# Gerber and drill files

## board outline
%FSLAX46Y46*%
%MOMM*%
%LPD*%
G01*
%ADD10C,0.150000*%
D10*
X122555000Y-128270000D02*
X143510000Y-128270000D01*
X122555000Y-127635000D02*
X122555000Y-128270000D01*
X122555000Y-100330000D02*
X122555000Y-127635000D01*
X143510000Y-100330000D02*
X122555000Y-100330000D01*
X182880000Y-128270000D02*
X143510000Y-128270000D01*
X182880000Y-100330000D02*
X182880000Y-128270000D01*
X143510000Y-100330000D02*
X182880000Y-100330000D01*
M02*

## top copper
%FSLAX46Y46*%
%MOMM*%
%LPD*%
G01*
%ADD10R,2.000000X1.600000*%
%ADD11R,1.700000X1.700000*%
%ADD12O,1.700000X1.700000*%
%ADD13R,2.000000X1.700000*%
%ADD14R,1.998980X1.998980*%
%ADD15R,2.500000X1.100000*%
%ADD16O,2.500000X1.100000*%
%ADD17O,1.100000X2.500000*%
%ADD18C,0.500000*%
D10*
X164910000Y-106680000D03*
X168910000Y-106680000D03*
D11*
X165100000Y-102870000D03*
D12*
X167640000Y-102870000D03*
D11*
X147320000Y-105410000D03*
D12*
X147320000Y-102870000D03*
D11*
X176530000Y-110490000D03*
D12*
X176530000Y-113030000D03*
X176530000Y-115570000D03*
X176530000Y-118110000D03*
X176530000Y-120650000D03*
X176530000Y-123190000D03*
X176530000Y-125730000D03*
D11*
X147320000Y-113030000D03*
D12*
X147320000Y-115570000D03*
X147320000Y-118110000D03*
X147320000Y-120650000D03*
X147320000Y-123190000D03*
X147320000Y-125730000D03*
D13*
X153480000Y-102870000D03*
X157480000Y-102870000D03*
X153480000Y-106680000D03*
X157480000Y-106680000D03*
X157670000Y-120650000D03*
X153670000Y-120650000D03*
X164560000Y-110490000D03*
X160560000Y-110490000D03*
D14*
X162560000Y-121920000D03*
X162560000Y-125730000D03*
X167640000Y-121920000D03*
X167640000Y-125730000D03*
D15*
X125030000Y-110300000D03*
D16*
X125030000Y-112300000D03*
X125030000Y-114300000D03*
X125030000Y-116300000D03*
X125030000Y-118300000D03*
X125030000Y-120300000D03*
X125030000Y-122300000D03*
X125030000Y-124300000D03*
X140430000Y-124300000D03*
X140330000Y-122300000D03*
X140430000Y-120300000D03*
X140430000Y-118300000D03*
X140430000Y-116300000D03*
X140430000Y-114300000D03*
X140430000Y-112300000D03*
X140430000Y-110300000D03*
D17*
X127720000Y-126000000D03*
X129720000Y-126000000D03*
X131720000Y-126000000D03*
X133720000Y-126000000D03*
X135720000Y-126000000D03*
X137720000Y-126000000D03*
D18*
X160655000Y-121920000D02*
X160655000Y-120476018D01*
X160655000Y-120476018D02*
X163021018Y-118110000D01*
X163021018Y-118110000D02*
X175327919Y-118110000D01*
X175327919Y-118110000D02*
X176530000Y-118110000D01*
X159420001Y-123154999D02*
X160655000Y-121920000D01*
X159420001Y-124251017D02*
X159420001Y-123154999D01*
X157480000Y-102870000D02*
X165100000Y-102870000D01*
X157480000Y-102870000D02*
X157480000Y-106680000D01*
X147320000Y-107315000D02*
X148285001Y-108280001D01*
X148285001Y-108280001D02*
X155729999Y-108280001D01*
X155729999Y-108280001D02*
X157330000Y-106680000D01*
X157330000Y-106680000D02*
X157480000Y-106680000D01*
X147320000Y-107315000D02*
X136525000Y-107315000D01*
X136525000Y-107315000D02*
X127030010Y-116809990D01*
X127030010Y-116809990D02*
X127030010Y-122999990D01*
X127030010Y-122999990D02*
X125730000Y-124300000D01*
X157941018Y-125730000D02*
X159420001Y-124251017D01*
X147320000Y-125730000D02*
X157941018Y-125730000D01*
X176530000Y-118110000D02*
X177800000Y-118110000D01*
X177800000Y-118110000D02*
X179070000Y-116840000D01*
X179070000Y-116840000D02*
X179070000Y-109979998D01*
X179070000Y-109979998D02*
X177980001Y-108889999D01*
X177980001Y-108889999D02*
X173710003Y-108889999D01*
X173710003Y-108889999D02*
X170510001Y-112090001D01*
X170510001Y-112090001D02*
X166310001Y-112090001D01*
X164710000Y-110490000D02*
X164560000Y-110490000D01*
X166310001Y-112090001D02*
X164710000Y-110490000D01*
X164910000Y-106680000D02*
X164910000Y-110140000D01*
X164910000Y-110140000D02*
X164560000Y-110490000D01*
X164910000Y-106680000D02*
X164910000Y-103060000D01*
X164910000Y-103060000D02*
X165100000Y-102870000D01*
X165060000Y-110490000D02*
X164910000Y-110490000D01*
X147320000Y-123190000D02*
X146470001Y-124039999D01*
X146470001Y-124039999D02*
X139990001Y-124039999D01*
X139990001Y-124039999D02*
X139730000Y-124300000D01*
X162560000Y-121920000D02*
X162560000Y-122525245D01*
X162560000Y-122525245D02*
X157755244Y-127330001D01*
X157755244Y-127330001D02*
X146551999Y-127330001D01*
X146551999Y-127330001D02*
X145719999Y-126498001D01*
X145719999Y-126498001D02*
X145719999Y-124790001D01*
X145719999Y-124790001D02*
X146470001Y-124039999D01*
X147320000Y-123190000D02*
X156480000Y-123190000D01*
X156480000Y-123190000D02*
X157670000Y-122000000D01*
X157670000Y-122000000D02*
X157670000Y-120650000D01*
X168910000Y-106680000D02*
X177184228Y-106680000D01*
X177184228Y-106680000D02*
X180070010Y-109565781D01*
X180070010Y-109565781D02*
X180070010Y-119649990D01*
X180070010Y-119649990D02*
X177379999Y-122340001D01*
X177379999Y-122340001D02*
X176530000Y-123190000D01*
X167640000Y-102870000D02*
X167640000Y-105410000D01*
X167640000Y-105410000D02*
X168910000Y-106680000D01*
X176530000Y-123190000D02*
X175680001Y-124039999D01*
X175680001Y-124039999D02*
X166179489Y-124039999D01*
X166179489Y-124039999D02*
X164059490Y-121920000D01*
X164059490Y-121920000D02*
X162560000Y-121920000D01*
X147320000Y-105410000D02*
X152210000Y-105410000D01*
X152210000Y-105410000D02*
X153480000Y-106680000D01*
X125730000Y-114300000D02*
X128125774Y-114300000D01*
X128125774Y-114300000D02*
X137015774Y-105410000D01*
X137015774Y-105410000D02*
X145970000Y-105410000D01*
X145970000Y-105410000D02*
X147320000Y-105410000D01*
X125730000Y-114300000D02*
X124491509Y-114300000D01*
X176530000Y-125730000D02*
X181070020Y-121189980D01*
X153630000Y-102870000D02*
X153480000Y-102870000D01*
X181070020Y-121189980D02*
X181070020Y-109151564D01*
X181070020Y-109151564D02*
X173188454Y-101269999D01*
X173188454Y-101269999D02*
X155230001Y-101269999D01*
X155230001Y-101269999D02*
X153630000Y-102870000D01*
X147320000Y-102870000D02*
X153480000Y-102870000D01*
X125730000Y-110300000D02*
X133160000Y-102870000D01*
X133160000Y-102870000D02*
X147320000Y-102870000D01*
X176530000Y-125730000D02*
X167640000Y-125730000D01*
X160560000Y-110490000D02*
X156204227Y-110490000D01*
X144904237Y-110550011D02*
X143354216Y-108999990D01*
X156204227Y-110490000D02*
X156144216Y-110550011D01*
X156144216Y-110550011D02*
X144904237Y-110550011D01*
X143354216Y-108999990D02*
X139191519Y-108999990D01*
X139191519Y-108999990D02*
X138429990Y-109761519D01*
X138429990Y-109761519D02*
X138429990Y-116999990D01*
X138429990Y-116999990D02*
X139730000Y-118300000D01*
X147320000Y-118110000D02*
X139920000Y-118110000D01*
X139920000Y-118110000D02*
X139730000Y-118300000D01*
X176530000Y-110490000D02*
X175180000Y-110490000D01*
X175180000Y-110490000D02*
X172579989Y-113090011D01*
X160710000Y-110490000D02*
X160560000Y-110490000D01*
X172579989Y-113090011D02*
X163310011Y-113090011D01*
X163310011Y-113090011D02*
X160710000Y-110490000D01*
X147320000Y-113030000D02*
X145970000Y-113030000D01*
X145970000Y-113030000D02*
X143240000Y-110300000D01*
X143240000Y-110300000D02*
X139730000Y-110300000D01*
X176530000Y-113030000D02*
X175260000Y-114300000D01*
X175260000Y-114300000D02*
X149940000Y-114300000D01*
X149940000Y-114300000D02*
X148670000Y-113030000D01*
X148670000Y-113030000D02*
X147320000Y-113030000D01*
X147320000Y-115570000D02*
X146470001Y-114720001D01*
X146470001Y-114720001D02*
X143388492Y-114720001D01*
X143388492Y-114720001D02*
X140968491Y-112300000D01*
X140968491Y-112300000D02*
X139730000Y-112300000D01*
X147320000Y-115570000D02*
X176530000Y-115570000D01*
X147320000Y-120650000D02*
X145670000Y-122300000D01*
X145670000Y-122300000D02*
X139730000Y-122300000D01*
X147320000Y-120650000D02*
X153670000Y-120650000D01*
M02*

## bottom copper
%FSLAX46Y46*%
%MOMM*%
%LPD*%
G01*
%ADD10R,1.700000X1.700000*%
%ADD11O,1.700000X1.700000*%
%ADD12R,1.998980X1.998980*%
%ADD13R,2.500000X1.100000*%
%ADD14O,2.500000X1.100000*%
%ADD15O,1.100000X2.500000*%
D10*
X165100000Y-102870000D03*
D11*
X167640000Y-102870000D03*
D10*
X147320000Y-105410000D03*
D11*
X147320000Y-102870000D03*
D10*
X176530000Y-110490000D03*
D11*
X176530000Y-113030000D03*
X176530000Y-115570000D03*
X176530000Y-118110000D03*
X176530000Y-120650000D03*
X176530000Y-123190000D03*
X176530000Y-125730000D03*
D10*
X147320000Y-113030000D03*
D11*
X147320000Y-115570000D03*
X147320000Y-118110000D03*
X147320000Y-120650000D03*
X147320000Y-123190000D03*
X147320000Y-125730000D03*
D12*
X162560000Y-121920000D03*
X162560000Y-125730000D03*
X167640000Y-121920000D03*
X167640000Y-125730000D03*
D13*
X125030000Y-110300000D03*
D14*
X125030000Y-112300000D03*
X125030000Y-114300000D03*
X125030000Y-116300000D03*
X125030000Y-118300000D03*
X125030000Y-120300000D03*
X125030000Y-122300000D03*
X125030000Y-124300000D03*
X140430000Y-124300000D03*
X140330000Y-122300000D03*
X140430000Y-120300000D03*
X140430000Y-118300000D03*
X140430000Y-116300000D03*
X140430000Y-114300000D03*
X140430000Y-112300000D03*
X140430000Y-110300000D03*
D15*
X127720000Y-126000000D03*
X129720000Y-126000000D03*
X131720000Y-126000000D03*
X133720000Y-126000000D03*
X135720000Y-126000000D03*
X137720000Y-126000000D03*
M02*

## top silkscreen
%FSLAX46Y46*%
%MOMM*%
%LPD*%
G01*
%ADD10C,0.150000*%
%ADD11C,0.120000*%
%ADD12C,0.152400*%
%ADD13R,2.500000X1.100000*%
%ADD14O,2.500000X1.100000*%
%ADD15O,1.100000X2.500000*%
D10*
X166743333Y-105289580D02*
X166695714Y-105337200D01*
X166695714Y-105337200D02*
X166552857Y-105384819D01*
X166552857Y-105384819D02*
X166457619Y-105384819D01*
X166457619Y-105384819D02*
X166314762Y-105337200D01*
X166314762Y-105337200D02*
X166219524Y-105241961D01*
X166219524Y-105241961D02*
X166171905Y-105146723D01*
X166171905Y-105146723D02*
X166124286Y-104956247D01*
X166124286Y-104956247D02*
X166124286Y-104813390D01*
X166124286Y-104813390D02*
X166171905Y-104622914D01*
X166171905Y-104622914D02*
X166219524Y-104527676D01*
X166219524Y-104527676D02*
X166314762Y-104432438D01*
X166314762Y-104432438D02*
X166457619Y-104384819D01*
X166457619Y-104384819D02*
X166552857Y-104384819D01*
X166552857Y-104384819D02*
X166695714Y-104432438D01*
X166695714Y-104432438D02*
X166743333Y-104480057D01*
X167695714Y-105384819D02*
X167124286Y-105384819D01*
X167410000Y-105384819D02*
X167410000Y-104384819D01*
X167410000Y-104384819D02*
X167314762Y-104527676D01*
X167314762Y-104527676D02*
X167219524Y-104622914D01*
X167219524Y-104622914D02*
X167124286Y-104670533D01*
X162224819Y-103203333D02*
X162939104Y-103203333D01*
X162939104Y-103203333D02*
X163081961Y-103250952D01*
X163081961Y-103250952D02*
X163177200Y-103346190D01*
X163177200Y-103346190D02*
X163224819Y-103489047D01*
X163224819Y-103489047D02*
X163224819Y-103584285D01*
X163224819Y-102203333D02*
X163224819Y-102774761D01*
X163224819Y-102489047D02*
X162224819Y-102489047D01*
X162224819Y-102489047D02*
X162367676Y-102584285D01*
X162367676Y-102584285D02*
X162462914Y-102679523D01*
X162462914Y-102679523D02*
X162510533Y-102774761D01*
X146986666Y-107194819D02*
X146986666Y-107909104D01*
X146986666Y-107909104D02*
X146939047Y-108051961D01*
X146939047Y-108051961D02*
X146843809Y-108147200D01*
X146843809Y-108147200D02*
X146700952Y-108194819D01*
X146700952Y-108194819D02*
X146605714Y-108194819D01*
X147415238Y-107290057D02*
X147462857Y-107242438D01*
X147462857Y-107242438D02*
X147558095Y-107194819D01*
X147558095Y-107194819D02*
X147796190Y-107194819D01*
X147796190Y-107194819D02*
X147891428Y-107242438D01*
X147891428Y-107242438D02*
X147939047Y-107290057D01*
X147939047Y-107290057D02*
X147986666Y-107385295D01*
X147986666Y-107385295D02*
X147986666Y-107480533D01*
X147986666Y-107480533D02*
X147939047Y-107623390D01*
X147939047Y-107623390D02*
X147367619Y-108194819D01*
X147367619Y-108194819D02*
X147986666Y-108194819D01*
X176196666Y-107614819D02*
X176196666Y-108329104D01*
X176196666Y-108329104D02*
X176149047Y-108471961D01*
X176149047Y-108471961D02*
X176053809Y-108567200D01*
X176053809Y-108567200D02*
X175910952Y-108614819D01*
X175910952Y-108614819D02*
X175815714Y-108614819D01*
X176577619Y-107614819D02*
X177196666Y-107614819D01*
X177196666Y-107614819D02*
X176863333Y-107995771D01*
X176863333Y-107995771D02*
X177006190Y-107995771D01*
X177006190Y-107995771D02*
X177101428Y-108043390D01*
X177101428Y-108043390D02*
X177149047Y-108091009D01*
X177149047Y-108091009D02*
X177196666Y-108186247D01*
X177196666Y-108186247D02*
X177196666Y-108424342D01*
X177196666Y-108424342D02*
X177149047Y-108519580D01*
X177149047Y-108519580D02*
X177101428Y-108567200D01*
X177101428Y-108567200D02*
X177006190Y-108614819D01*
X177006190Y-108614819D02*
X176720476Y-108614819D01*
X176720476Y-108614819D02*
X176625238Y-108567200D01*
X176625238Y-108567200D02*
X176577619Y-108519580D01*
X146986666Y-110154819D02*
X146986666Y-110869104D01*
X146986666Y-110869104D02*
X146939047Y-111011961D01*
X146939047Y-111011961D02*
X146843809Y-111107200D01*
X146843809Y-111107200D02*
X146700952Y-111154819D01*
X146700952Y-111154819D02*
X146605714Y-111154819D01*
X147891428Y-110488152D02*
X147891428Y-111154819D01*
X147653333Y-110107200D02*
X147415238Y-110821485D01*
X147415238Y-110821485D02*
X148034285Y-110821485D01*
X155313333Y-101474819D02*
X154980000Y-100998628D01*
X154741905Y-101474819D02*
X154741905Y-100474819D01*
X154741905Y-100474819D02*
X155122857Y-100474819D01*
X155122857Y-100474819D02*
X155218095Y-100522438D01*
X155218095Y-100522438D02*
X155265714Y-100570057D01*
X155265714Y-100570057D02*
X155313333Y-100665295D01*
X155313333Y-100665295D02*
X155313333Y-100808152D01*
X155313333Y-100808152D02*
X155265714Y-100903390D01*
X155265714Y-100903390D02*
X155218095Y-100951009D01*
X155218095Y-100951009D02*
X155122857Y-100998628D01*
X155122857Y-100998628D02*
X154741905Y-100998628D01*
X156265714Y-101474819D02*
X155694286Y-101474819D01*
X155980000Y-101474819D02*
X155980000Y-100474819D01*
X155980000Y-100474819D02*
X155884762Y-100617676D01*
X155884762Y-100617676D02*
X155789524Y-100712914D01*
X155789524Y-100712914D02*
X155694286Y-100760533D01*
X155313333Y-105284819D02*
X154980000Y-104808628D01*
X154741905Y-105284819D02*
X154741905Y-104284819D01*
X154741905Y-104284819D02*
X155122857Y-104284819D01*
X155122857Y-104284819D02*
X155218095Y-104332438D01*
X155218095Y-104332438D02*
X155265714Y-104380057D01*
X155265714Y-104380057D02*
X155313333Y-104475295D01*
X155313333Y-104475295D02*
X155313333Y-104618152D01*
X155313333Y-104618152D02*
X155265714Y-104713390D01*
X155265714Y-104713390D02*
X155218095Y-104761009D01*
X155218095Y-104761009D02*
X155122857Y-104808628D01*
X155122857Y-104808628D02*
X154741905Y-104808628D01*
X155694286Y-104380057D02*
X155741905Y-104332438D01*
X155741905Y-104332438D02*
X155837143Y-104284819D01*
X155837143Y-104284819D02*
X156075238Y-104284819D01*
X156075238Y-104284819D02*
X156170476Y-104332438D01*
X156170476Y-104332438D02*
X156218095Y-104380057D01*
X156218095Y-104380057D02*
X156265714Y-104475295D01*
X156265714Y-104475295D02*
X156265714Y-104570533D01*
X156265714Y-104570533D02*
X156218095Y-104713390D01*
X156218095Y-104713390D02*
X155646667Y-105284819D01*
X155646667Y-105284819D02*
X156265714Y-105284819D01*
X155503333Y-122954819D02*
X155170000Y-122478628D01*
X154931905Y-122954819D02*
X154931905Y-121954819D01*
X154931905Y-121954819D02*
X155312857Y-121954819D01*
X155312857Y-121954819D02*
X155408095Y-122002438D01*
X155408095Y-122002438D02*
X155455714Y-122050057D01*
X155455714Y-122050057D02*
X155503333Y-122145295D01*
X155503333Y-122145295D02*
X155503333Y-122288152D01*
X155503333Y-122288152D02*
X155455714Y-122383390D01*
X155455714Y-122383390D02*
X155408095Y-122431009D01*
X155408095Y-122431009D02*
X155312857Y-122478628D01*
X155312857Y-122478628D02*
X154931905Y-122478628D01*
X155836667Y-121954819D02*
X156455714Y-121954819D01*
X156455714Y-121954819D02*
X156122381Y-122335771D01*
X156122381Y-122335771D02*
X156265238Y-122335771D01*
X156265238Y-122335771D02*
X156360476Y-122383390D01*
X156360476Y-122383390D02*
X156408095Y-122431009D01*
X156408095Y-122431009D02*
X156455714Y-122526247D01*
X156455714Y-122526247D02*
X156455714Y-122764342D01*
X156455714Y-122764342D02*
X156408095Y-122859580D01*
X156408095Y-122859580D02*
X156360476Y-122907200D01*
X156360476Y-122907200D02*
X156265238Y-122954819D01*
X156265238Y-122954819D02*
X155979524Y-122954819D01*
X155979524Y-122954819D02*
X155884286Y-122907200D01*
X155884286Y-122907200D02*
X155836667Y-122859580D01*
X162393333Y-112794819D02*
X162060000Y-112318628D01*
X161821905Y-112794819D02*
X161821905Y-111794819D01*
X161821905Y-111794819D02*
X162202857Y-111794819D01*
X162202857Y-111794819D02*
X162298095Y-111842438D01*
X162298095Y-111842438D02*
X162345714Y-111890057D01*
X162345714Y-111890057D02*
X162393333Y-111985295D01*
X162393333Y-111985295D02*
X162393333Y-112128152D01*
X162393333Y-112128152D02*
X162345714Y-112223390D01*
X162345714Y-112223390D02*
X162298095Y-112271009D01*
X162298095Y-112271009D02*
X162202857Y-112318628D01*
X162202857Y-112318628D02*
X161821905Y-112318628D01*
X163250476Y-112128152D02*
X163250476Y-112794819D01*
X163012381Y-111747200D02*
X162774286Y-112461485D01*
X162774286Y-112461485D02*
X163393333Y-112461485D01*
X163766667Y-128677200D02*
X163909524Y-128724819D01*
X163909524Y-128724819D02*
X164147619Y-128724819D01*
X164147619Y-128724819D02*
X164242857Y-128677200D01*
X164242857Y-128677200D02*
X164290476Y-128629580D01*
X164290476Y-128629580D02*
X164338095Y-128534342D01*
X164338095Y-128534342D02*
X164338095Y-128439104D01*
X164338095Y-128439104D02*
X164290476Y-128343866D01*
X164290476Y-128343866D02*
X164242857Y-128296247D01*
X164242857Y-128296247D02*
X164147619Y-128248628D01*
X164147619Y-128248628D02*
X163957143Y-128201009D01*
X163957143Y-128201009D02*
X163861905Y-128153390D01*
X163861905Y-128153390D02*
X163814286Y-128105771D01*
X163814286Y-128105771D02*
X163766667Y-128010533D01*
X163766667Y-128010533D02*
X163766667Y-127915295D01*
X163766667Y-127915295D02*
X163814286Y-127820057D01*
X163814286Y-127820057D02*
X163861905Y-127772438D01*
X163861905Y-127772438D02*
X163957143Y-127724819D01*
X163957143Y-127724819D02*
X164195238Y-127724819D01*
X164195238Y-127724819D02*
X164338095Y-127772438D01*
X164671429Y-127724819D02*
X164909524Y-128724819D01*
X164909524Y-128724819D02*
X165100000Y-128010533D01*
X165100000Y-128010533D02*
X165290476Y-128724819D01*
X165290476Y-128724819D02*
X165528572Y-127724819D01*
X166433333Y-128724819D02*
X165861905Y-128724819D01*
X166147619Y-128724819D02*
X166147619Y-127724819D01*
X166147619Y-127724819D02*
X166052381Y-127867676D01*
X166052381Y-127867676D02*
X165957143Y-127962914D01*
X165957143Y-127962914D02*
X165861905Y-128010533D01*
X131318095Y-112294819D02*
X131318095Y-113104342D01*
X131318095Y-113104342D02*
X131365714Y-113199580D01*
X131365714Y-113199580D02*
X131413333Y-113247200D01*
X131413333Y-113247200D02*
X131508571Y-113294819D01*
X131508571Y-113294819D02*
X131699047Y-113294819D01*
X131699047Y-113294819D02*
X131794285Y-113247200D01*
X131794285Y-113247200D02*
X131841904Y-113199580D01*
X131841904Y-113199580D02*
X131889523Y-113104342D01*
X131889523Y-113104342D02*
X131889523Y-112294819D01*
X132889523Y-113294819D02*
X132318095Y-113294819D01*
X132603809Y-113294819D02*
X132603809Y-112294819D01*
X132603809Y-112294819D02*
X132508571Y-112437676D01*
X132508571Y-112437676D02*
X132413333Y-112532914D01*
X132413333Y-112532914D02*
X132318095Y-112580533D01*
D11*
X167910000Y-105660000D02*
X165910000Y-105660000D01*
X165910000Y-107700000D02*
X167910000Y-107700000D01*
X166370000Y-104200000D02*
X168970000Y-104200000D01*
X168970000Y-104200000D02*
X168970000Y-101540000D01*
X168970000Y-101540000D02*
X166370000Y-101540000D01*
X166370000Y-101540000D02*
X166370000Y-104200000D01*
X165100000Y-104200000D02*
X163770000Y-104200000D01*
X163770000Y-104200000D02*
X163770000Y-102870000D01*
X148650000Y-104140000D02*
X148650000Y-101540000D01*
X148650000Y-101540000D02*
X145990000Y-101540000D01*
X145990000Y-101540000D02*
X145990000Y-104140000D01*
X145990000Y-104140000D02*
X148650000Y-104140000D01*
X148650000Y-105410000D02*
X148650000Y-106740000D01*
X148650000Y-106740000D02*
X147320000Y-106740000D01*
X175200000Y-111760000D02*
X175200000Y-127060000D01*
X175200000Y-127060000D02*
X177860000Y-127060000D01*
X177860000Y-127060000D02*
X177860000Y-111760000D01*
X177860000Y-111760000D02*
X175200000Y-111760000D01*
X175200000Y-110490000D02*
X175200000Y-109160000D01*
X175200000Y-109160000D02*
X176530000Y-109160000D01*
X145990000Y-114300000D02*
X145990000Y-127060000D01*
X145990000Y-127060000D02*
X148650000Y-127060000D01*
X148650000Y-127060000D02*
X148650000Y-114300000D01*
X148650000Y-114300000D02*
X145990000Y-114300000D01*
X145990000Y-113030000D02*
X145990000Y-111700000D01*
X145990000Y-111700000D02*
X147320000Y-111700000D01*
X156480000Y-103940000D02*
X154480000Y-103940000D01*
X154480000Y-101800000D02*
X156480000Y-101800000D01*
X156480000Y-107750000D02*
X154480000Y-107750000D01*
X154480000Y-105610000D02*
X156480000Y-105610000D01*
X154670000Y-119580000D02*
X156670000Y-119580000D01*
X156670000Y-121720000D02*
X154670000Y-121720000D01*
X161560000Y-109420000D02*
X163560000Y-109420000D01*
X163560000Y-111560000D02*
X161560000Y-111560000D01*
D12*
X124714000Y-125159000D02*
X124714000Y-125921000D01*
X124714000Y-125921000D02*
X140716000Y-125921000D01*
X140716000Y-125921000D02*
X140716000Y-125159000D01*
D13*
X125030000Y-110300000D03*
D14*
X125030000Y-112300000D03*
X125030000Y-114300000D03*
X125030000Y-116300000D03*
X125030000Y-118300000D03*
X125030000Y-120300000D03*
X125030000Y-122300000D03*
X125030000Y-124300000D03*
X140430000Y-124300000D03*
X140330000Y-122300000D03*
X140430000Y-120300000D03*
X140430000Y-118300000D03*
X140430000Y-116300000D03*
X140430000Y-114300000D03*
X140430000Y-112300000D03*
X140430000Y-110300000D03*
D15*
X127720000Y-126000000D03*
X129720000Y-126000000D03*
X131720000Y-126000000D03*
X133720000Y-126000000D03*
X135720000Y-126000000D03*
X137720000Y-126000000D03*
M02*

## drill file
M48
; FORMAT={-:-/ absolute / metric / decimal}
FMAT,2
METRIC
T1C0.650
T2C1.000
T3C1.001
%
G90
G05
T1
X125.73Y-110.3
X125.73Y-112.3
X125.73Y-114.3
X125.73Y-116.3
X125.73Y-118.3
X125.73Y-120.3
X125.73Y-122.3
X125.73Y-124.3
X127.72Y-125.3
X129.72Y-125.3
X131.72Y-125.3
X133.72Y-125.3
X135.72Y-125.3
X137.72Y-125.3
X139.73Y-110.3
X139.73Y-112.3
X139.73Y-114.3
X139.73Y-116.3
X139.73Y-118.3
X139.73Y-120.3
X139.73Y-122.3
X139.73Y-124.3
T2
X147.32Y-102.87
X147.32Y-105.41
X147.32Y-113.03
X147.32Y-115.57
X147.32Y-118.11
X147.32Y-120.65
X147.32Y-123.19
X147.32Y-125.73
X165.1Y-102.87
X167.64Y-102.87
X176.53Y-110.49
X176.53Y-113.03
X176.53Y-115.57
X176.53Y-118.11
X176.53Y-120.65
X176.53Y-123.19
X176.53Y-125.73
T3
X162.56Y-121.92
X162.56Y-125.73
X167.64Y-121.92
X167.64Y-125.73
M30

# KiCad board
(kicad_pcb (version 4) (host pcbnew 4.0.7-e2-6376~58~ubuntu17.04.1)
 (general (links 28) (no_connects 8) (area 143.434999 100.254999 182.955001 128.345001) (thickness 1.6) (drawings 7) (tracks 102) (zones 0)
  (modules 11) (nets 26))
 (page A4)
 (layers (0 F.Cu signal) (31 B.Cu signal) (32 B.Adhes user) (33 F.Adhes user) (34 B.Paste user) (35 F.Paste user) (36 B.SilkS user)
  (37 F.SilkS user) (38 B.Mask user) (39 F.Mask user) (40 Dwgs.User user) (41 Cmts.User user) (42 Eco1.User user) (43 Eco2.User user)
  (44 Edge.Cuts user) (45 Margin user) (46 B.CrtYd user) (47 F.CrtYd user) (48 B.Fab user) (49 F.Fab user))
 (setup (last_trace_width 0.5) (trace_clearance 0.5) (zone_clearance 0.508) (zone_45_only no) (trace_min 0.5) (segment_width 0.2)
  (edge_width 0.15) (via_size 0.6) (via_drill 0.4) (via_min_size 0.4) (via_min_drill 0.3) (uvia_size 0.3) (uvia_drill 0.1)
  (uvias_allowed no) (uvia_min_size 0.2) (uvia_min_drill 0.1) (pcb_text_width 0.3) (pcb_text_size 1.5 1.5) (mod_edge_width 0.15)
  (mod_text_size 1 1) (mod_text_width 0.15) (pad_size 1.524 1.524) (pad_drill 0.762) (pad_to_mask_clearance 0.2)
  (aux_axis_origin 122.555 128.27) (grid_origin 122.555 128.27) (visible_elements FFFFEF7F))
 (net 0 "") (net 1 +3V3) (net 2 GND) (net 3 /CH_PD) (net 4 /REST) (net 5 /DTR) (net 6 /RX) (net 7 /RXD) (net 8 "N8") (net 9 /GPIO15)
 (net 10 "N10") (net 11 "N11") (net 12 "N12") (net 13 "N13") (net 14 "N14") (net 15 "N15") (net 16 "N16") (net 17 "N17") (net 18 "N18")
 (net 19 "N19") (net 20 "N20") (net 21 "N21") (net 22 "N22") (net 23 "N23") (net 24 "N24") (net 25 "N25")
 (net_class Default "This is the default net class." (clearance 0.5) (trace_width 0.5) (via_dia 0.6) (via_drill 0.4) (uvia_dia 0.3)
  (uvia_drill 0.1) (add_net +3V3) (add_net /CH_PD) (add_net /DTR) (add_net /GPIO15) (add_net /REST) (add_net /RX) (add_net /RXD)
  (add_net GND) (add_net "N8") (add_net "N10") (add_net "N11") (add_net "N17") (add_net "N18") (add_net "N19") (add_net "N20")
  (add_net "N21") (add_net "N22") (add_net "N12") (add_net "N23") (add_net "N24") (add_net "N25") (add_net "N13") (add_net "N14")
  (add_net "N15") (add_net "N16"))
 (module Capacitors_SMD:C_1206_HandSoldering (layer F.Cu) (at 166.91 106.68)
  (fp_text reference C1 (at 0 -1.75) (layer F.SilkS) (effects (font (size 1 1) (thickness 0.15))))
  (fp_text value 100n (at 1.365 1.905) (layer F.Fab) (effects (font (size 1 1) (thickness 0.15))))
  (fp_line (start 1 -1.02) (end -1 -1.02) (layer F.SilkS) (width 0.12))
  (fp_line (start -1 1.02) (end 1 1.02) (layer F.SilkS) (width 0.12))
  (pad 1 smd rect (at -2 0) (size 2 1.6) (layers F.Cu F.Paste F.Mask) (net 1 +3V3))
  (pad 2 smd rect (at 2 0) (size 2 1.6) (layers F.Cu F.Paste F.Mask) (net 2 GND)))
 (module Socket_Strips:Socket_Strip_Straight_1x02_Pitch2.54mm (layer F.Cu) (at 165.1 102.87 90)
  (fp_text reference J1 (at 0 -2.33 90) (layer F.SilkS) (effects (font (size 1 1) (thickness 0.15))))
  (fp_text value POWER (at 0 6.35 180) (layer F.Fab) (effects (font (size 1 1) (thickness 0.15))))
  (fp_line (start -1.33 1.27) (end -1.33 3.87) (layer F.SilkS) (width 0.12))
  (fp_line (start -1.33 3.87) (end 1.33 3.87) (layer F.SilkS) (width 0.12))
  (fp_line (start 1.33 3.87) (end 1.33 1.27) (layer F.SilkS) (width 0.12))
  (fp_line (start 1.33 1.27) (end -1.33 1.27) (layer F.SilkS) (width 0.12))
  (fp_line (start -1.33 0) (end -1.33 -1.33) (layer F.SilkS) (width 0.12))
  (fp_line (start -1.33 -1.33) (end 0 -1.33) (layer F.SilkS) (width 0.12))
  (pad 1 thru_hole rect (at 0 0 90) (size 1.7 1.7) (drill 1) (layers *.Cu *.Mask) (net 1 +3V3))
  (pad 2 thru_hole oval (at 0 2.54 90) (size 1.7 1.7) (drill 1) (layers *.Cu *.Mask) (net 2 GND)))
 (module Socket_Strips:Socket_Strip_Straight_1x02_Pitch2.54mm (layer F.Cu) (at 147.32 105.41 180)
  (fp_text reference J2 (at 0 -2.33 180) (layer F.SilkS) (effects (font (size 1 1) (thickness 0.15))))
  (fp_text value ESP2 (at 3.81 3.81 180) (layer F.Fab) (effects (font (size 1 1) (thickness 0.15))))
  (fp_line (start -1.33 1.27) (end -1.33 3.87) (layer F.SilkS) (width 0.12))
  (fp_line (start -1.33 3.87) (end 1.33 3.87) (layer F.SilkS) (width 0.12))
  (fp_line (start 1.33 3.87) (end 1.33 1.27) (layer F.SilkS) (width 0.12))
  (fp_line (start 1.33 1.27) (end -1.33 1.27) (layer F.SilkS) (width 0.12))
  (fp_line (start -1.33 0) (end -1.33 -1.33) (layer F.SilkS) (width 0.12))
  (fp_line (start -1.33 -1.33) (end 0 -1.33) (layer F.SilkS) (width 0.12))
  (pad 1 thru_hole rect (at 0 0 180) (size 1.7 1.7) (drill 1) (layers *.Cu *.Mask) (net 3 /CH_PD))
  (pad 2 thru_hole oval (at 0 2.54 180) (size 1.7 1.7) (drill 1) (layers *.Cu *.Mask) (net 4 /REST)))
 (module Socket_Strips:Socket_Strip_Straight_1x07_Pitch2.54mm (layer F.Cu) (at 176.53 110.49)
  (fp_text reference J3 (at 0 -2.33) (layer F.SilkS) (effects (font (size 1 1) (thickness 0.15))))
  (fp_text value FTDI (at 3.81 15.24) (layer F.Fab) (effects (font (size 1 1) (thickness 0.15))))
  (fp_line (start -1.33 1.27) (end -1.33 16.57) (layer F.SilkS) (width 0.12))
  (fp_line (start -1.33 16.57) (end 1.33 16.57) (layer F.SilkS) (width 0.12))
  (fp_line (start 1.33 16.57) (end 1.33 1.27) (layer F.SilkS) (width 0.12))
  (fp_line (start 1.33 1.27) (end -1.33 1.27) (layer F.SilkS) (width 0.12))
  (fp_line (start -1.33 0) (end -1.33 -1.33) (layer F.SilkS) (width 0.12))
  (fp_line (start -1.33 -1.33) (end 0 -1.33) (layer F.SilkS) (width 0.12))
  (pad 1 thru_hole rect (at 0 0) (size 1.7 1.7) (drill 1) (layers *.Cu *.Mask) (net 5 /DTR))
  (pad 2 thru_hole oval (at 0 2.54) (size 1.7 1.7) (drill 1) (layers *.Cu *.Mask) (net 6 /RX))
  (pad 3 thru_hole oval (at 0 5.08) (size 1.7 1.7) (drill 1) (layers *.Cu *.Mask) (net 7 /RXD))
  (pad 4 thru_hole oval (at 0 7.62) (size 1.7 1.7) (drill 1) (layers *.Cu *.Mask) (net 1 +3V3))
  (pad 5 thru_hole oval (at 0 10.16) (size 1.7 1.7) (drill 1) (layers *.Cu *.Mask) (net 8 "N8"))
  (pad 6 thru_hole oval (at 0 12.7) (size 1.7 1.7) (drill 1) (layers *.Cu *.Mask) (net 2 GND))
  (pad 7 thru_hole oval (at 0 15.24) (size 1.7 1.7) (drill 1) (layers *.Cu *.Mask) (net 4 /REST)))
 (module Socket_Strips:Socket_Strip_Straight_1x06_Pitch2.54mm (layer F.Cu) (at 147.32 113.03)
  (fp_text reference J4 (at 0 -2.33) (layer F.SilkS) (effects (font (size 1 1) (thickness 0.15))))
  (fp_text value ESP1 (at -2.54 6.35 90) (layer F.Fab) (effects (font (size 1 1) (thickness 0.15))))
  (fp_line (start -1.33 1.27) (end -1.33 14.03) (layer F.SilkS) (width 0.12))
  (fp_line (start -1.33 14.03) (end 1.33 14.03) (layer F.SilkS) (width 0.12))
  (fp_line (start 1.33 14.03) (end 1.33 1.27) (layer F.SilkS) (width 0.12))
  (fp_line (start 1.33 1.27) (end -1.33 1.27) (layer F.SilkS) (width 0.12))
  (fp_line (start -1.33 0) (end -1.33 -1.33) (layer F.SilkS) (width 0.12))
  (fp_line (start -1.33 -1.33) (end 0 -1.33) (layer F.SilkS) (width 0.12))
  (pad 1 thru_hole rect (at 0 0) (size 1.7 1.7) (drill 1) (layers *.Cu *.Mask) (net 6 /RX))
  (pad 2 thru_hole oval (at 0 2.54) (size 1.7 1.7) (drill 1) (layers *.Cu *.Mask) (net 7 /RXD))
  (pad 3 thru_hole oval (at 0 5.08) (size 1.7 1.7) (drill 1) (layers *.Cu *.Mask) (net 5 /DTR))
  (pad 4 thru_hole oval (at 0 7.62) (size 1.7 1.7) (drill 1) (layers *.Cu *.Mask) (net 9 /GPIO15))
  (pad 5 thru_hole oval (at 0 10.16) (size 1.7 1.7) (drill 1) (layers *.Cu *.Mask) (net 2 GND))
  (pad 6 thru_hole oval (at 0 12.7) (size 1.7 1.7) (drill 1) (layers *.Cu *.Mask) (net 1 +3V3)))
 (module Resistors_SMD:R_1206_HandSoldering (layer F.Cu) (at 155.48 102.87)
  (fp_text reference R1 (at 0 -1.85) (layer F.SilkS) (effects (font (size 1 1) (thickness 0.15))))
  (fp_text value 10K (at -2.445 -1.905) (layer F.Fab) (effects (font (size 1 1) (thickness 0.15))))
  (fp_line (start 1 1.07) (end -1 1.07) (layer F.SilkS) (width 0.12))
  (fp_line (start -1 -1.07) (end 1 -1.07) (layer F.SilkS) (width 0.12))
  (pad 1 smd rect (at -2 0) (size 2 1.7) (layers F.Cu F.Paste F.Mask) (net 4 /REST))
  (pad 2 smd rect (at 2 0) (size 2 1.7) (layers F.Cu F.Paste F.Mask) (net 1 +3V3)))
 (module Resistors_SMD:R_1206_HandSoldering (layer F.Cu) (at 155.48 106.68)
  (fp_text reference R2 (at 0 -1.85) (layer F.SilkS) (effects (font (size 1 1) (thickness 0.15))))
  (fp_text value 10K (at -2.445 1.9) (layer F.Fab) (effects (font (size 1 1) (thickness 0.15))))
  (fp_line (start 1 1.07) (end -1 1.07) (layer F.SilkS) (width 0.12))
  (fp_line (start -1 -1.07) (end 1 -1.07) (layer F.SilkS) (width 0.12))
  (pad 1 smd rect (at -2 0) (size 2 1.7) (layers F.Cu F.Paste F.Mask) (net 3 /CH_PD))
  (pad 2 smd rect (at 2 0) (size 2 1.7) (layers F.Cu F.Paste F.Mask) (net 1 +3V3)))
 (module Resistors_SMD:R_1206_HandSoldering (layer F.Cu) (at 155.67 120.65 180)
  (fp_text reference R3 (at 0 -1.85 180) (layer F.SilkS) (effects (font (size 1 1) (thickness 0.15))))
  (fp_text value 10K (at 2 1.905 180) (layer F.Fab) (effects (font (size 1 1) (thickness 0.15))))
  (fp_line (start 1 1.07) (end -1 1.07) (layer F.SilkS) (width 0.12))
  (fp_line (start -1 -1.07) (end 1 -1.07) (layer F.SilkS) (width 0.12))
  (pad 1 smd rect (at -2 0 180) (size 2 1.7) (layers F.Cu F.Paste F.Mask) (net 2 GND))
  (pad 2 smd rect (at 2 0 180) (size 2 1.7) (layers F.Cu F.Paste F.Mask) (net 9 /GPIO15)))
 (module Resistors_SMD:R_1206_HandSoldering (layer F.Cu) (at 162.56 110.49 180)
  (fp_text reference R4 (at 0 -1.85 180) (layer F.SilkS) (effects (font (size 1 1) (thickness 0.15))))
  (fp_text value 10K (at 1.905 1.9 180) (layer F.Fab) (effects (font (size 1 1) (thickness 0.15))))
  (fp_line (start 1 1.07) (end -1 1.07) (layer F.SilkS) (width 0.12))
  (fp_line (start -1 -1.07) (end 1 -1.07) (layer F.SilkS) (width 0.12))
  (pad 1 smd rect (at -2 0 180) (size 2 1.7) (layers F.Cu F.Paste F.Mask) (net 1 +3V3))
  (pad 2 smd rect (at 2 0 180) (size 2 1.7) (layers F.Cu F.Paste F.Mask) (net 5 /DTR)))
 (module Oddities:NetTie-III (layer F.Cu) (at 165.1 123.825)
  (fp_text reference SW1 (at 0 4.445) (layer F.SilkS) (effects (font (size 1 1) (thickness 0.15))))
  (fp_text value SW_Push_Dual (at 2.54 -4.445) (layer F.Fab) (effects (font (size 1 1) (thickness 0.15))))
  (pad 1 thru_hole rect (at -2.54 -1.905) (size 1.99898 1.99898) (drill 1.00076) (layers *.Cu *.Mask) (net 2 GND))
  (pad 2 thru_hole rect (at -2.54 1.905) (size 1.99898 1.99898) (drill 1.00076) (layers *.Cu *.Mask) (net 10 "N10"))
  (pad 3 thru_hole rect (at 2.54 -1.905) (size 1.99898 1.99898) (drill 1.00076) (layers *.Cu *.Mask) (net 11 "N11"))
  (pad 4 thru_hole rect (at 2.54 1.905) (size 1.99898 1.99898) (drill 1.00076) (layers *.Cu *.Mask) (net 4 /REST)))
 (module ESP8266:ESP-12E (layer F.Cu) (at 125.73 110.3)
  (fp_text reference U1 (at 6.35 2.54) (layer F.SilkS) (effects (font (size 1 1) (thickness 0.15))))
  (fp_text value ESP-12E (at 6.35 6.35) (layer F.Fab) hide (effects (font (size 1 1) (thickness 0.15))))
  (fp_line (start -1.016 14.859) (end -1.016 15.621) (layer F.SilkS) (width 0.1524))
  (fp_line (start -1.016 15.621) (end 14.986 15.621) (layer F.SilkS) (width 0.1524))
  (fp_line (start 14.986 15.621) (end 14.986 14.859) (layer F.SilkS) (width 0.1524))
  (pad 1 thru_hole rect (at 0 0) (size 2.5 1.1) (drill 0.65 (offset -0.7 0)) (layers *.Cu *.Mask F.SilkS) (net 4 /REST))
  (pad 2 thru_hole oval (at 0 2) (size 2.5 1.1) (drill 0.65 (offset -0.7 0)) (layers *.Cu *.Mask F.SilkS) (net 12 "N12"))
  (pad 3 thru_hole oval (at 0 4) (size 2.5 1.1) (drill 0.65 (offset -0.7 0)) (layers *.Cu *.Mask F.SilkS) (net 3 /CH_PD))
  (pad 4 thru_hole oval (at 0 6) (size 2.5 1.1) (drill 0.65 (offset -0.7 0)) (layers *.Cu *.Mask F.SilkS) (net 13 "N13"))
  (pad 5 thru_hole oval (at 0 8) (size 2.5 1.1) (drill 0.65 (offset -0.7 0)) (layers *.Cu *.Mask F.SilkS) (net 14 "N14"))
  (pad 6 thru_hole oval (at 0 10) (size 2.5 1.1) (drill 0.65 (offset -0.7 0)) (layers *.Cu *.Mask F.SilkS) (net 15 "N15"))
  (pad 7 thru_hole oval (at 0 12) (size 2.5 1.1) (drill 0.65 (offset -0.7 0)) (layers *.Cu *.Mask F.SilkS) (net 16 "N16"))
  (pad 8 thru_hole oval (at 0 14) (size 2.5 1.1) (drill 0.65 (offset -0.7 0)) (layers *.Cu *.Mask F.SilkS) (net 1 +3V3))
  (pad 9 thru_hole oval (at 14 14) (size 2.5 1.1) (drill 0.65 (offset 0.7 0)) (layers *.Cu *.Mask F.SilkS) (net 2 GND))
  (pad 10 thru_hole oval (at 14 12) (size 2.5 1.1) (drill 0.65 (offset 0.6 0)) (layers *.Cu *.Mask F.SilkS) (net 9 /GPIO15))
  (pad 11 thru_hole oval (at 14 10) (size 2.5 1.1) (drill 0.65 (offset 0.7 0)) (layers *.Cu *.Mask F.SilkS) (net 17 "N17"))
  (pad 12 thru_hole oval (at 14 8) (size 2.5 1.1) (drill 0.65 (offset 0.7 0)) (layers *.Cu *.Mask F.SilkS) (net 5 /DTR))
  (pad 13 thru_hole oval (at 14 6) (size 2.5 1.1) (drill 0.65 (offset 0.7 0)) (layers *.Cu *.Mask F.SilkS) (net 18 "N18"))
  (pad 14 thru_hole oval (at 14 4) (size 2.5 1.1) (drill 0.65 (offset 0.7 0)) (layers *.Cu *.Mask F.SilkS) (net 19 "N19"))
  (pad 15 thru_hole oval (at 14 2) (size 2.5 1.1) (drill 0.65 (offset 0.7 0)) (layers *.Cu *.Mask F.SilkS) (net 7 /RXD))
  (pad 16 thru_hole oval (at 14 0) (size 2.5 1.1) (drill 0.65 (offset 0.7 0)) (layers *.Cu *.Mask F.SilkS) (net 6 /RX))
  (pad 17 thru_hole oval (at 1.99 15 90) (size 2.5 1.1) (drill 0.65 (offset -0.7 0)) (layers *.Cu *.Mask F.SilkS) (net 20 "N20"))
  (pad 18 thru_hole oval (at 3.99 15 90) (size 2.5 1.1) (drill 0.65 (offset -0.7 0)) (layers *.Cu *.Mask F.SilkS) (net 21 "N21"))
  (pad 19 thru_hole oval (at 5.99 15 90) (size 2.5 1.1) (drill 0.65 (offset -0.7 0)) (layers *.Cu *.Mask F.SilkS) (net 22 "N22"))
  (pad 20 thru_hole oval (at 7.99 15 90) (size 2.5 1.1) (drill 0.65 (offset -0.7 0)) (layers *.Cu *.Mask F.SilkS) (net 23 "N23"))
  (pad 21 thru_hole oval (at 9.99 15 90) (size 2.5 1.1) (drill 0.65 (offset -0.7 0)) (layers *.Cu *.Mask F.SilkS) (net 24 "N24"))
  (pad 22 thru_hole oval (at 11.99 15 90) (size 2.5 1.1) (drill 0.65 (offset -0.7 0)) (layers *.Cu *.Mask F.SilkS) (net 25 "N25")))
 (gr_line (start 122.555 128.27) (end 143.51 128.27) (layer Edge.Cuts) (width 0.15))
 (gr_line (start 122.555 127.635) (end 122.555 128.27) (layer Edge.Cuts) (width 0.15))
 (gr_line (start 122.555 100.33) (end 122.555 127.635) (layer Edge.Cuts) (width 0.15))
 (gr_line (start 143.51 100.33) (end 122.555 100.33) (layer Edge.Cuts) (width 0.15))
 (gr_line (start 182.88 128.27) (end 143.51 128.27) (layer Edge.Cuts) (width 0.15))
 (gr_line (start 182.88 100.33) (end 182.88 128.27) (layer Edge.Cuts) (width 0.15))
 (gr_line (start 143.51 100.33) (end 182.88 100.33) (layer Edge.Cuts) (width 0.15))
 (segment (start 160.655 121.92) (end 160.655 120.476018) (width 0.5) (layer F.Cu) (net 1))
 (segment (start 160.655 120.476018) (end 163.021018 118.11) (width 0.5) (layer F.Cu) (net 1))
 (segment (start 163.021018 118.11) (end 175.327919 118.11) (width 0.5) (layer F.Cu) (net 1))
 (segment (start 175.327919 118.11) (end 176.53 118.11) (width 0.5) (layer F.Cu) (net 1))
 (segment (start 159.420001 123.154999) (end 160.655 121.92) (width 0.5) (layer F.Cu) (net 1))
 (segment (start 159.420001 124.251017) (end 159.420001 123.154999) (width 0.5) (layer F.Cu) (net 1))
 (segment (start 157.48 102.87) (end 165.1 102.87) (width 0.5) (layer F.Cu) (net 1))
 (segment (start 157.48 102.87) (end 157.48 106.68) (width 0.5) (layer F.Cu) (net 1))
 (segment (start 147.32 107.315) (end 148.285001 108.280001) (width 0.5) (layer F.Cu) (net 1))
 (segment (start 148.285001 108.280001) (end 155.729999 108.280001) (width 0.5) (layer F.Cu) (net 1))
 (segment (start 155.729999 108.280001) (end 157.33 106.68) (width 0.5) (layer F.Cu) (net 1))
 (segment (start 157.33 106.68) (end 157.48 106.68) (width 0.5) (layer F.Cu) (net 1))
 (segment (start 147.32 107.315) (end 136.525 107.315) (width 0.5) (layer F.Cu) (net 1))
 (segment (start 136.525 107.315) (end 127.03001 116.80999) (width 0.5) (layer F.Cu) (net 1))
 (segment (start 127.03001 116.80999) (end 127.03001 122.99999) (width 0.5) (layer F.Cu) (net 1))
 (segment (start 127.03001 122.99999) (end 125.73 124.3) (width 0.5) (layer F.Cu) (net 1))
 (segment (start 157.941018 125.73) (end 159.420001 124.251017) (width 0.5) (layer F.Cu) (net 1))
 (segment (start 147.32 125.73) (end 157.941018 125.73) (width 0.5) (layer F.Cu) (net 1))
 (segment (start 176.53 118.11) (end 177.8 118.11) (width 0.5) (layer F.Cu) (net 1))
 (segment (start 177.8 118.11) (end 179.07 116.84) (width 0.5) (layer F.Cu) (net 1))
 (segment (start 179.07 116.84) (end 179.07 109.979998) (width 0.5) (layer F.Cu) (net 1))
 (segment (start 179.07 109.979998) (end 177.980001 108.889999) (width 0.5) (layer F.Cu) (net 1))
 (segment (start 177.980001 108.889999) (end 173.710003 108.889999) (width 0.5) (layer F.Cu) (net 1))
 (segment (start 173.710003 108.889999) (end 170.510001 112.090001) (width 0.5) (layer F.Cu) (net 1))
 (segment (start 170.510001 112.090001) (end 166.310001 112.090001) (width 0.5) (layer F.Cu) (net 1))
 (segment (start 164.71 110.49) (end 164.56 110.49) (width 0.5) (layer F.Cu) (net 1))
 (segment (start 166.310001 112.090001) (end 164.71 110.49) (width 0.5) (layer F.Cu) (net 1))
 (segment (start 164.91 106.68) (end 164.91 110.14) (width 0.5) (layer F.Cu) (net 1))
 (segment (start 164.91 110.14) (end 164.56 110.49) (width 0.5) (layer F.Cu) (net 1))
 (segment (start 164.91 106.68) (end 164.91 103.06) (width 0.5) (layer F.Cu) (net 1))
 (segment (start 164.91 103.06) (end 165.1 102.87) (width 0.5) (layer F.Cu) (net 1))
 (segment (start 165.06 110.49) (end 164.91 110.49) (width 0.5) (layer F.Cu) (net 1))
 (segment (start 147.32 123.19) (end 146.470001 124.039999) (width 0.5) (layer F.Cu) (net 2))
 (segment (start 146.470001 124.039999) (end 139.990001 124.039999) (width 0.5) (layer F.Cu) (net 2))
 (segment (start 139.990001 124.039999) (end 139.73 124.3) (width 0.5) (layer F.Cu) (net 2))
 (segment (start 162.56 121.92) (end 162.56 122.525245) (width 0.5) (layer F.Cu) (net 2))
 (segment (start 162.56 122.525245) (end 157.755244 127.330001) (width 0.5) (layer F.Cu) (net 2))
 (segment (start 157.755244 127.330001) (end 146.551999 127.330001) (width 0.5) (layer F.Cu) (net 2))
 (segment (start 146.551999 127.330001) (end 145.719999 126.498001) (width 0.5) (layer F.Cu) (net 2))
 (segment (start 145.719999 126.498001) (end 145.719999 124.790001) (width 0.5) (layer F.Cu) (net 2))
 (segment (start 145.719999 124.790001) (end 146.470001 124.039999) (width 0.5) (layer F.Cu) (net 2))
 (segment (start 147.32 123.19) (end 156.48 123.19) (width 0.5) (layer F.Cu) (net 2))
 (segment (start 156.48 123.19) (end 157.67 122) (width 0.5) (layer F.Cu) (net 2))
 (segment (start 157.67 122) (end 157.67 120.65) (width 0.5) (layer F.Cu) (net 2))
 (segment (start 168.91 106.68) (end 177.184228 106.68) (width 0.5) (layer F.Cu) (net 2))
 (segment (start 177.184228 106.68) (end 180.07001 109.565781) (width 0.5) (layer F.Cu) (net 2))
 (segment (start 180.07001 109.565781) (end 180.07001 119.64999) (width 0.5) (layer F.Cu) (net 2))
 (segment (start 180.07001 119.64999) (end 177.379999 122.340001) (width 0.5) (layer F.Cu) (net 2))
 (segment (start 177.379999 122.340001) (end 176.53 123.19) (width 0.5) (layer F.Cu) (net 2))
 (segment (start 167.64 102.87) (end 167.64 105.41) (width 0.5) (layer F.Cu) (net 2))
 (segment (start 167.64 105.41) (end 168.91 106.68) (width 0.5) (layer F.Cu) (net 2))
 (segment (start 176.53 123.19) (end 175.680001 124.039999) (width 0.5) (layer F.Cu) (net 2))
 (segment (start 175.680001 124.039999) (end 166.179489 124.039999) (width 0.5) (layer F.Cu) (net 2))
 (segment (start 166.179489 124.039999) (end 164.05949 121.92) (width 0.5) (layer F.Cu) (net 2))
 (segment (start 164.05949 121.92) (end 162.56 121.92) (width 0.5) (layer F.Cu) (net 2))
 (segment (start 147.32 105.41) (end 152.21 105.41) (width 0.5) (layer F.Cu) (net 3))
 (segment (start 152.21 105.41) (end 153.48 106.68) (width 0.5) (layer F.Cu) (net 3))
 (segment (start 125.73 114.3) (end 128.125774 114.3) (width 0.5) (layer F.Cu) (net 3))
 (segment (start 128.125774 114.3) (end 137.015774 105.41) (width 0.5) (layer F.Cu) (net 3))
 (segment (start 137.015774 105.41) (end 145.97 105.41) (width 0.5) (layer F.Cu) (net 3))
 (segment (start 145.97 105.41) (end 147.32 105.41) (width 0.5) (layer F.Cu) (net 3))
 (segment (start 125.73 114.3) (end 124.491509 114.3) (width 0.5) (layer F.Cu) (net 3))
 (segment (start 176.53 125.73) (end 181.07002 121.18998) (width 0.5) (layer F.Cu) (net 4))
 (segment (start 153.63 102.87) (end 153.48 102.87) (width 0.5) (layer F.Cu) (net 4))
 (segment (start 181.07002 121.18998) (end 181.07002 109.151564) (width 0.5) (layer F.Cu) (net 4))
 (segment (start 181.07002 109.151564) (end 173.188454 101.269999) (width 0.5) (layer F.Cu) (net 4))
 (segment (start 173.188454 101.269999) (end 155.230001 101.269999) (width 0.5) (layer F.Cu) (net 4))
 (segment (start 155.230001 101.269999) (end 153.63 102.87) (width 0.5) (layer F.Cu) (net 4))
 (segment (start 147.32 102.87) (end 153.48 102.87) (width 0.5) (layer F.Cu) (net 4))
 (segment (start 125.73 110.3) (end 133.16 102.87) (width 0.5) (layer F.Cu) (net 4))
 (segment (start 133.16 102.87) (end 147.32 102.87) (width 0.5) (layer F.Cu) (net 4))
 (segment (start 176.53 125.73) (end 167.64 125.73) (width 0.5) (layer F.Cu) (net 4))
 (segment (start 160.56 110.49) (end 156.204227 110.49) (width 0.5) (layer F.Cu) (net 5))
 (segment (start 144.904237 110.550011) (end 143.354216 108.99999) (width 0.5) (layer F.Cu) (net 5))
 (segment (start 156.204227 110.49) (end 156.144216 110.550011) (width 0.5) (layer F.Cu) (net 5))
 (segment (start 156.144216 110.550011) (end 144.904237 110.550011) (width 0.5) (layer F.Cu) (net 5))
 (segment (start 143.354216 108.99999) (end 139.191519 108.99999) (width 0.5) (layer F.Cu) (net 5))
 (segment (start 139.191519 108.99999) (end 138.42999 109.761519) (width 0.5) (layer F.Cu) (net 5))
 (segment (start 138.42999 109.761519) (end 138.42999 116.99999) (width 0.5) (layer F.Cu) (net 5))
 (segment (start 138.42999 116.99999) (end 139.73 118.3) (width 0.5) (layer F.Cu) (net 5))
 (segment (start 147.32 118.11) (end 139.92 118.11) (width 0.5) (layer F.Cu) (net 5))
 (segment (start 139.92 118.11) (end 139.73 118.3) (width 0.5) (layer F.Cu) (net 5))
 (segment (start 176.53 110.49) (end 175.18 110.49) (width 0.5) (layer F.Cu) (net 5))
 (segment (start 175.18 110.49) (end 172.579989 113.090011) (width 0.5) (layer F.Cu) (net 5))
 (segment (start 160.71 110.49) (end 160.56 110.49) (width 0.5) (layer F.Cu) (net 5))
 (segment (start 172.579989 113.090011) (end 163.310011 113.090011) (width 0.5) (layer F.Cu) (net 5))
 (segment (start 163.310011 113.090011) (end 160.71 110.49) (width 0.5) (layer F.Cu) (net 5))
 (segment (start 147.32 113.03) (end 145.97 113.03) (width 0.5) (layer F.Cu) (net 6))
 (segment (start 145.97 113.03) (end 143.24 110.3) (width 0.5) (layer F.Cu) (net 6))
 (segment (start 143.24 110.3) (end 139.73 110.3) (width 0.5) (layer F.Cu) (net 6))
 (segment (start 176.53 113.03) (end 175.26 114.3) (width 0.5) (layer F.Cu) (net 6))
 (segment (start 175.26 114.3) (end 149.94 114.3) (width 0.5) (layer F.Cu) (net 6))
 (segment (start 149.94 114.3) (end 148.67 113.03) (width 0.5) (layer F.Cu) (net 6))
 (segment (start 148.67 113.03) (end 147.32 113.03) (width 0.5) (layer F.Cu) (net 6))
 (segment (start 147.32 115.57) (end 146.470001 114.720001) (width 0.5) (layer F.Cu) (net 7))
 (segment (start 146.470001 114.720001) (end 143.388492 114.720001) (width 0.5) (layer F.Cu) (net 7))
 (segment (start 143.388492 114.720001) (end 140.968491 112.3) (width 0.5) (layer F.Cu) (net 7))
 (segment (start 140.968491 112.3) (end 139.73 112.3) (width 0.5) (layer F.Cu) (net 7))
 (segment (start 147.32 115.57) (end 176.53 115.57) (width 0.5) (layer F.Cu) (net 7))
 (segment (start 147.32 120.65) (end 145.67 122.3) (width 0.5) (layer F.Cu) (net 9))
 (segment (start 145.67 122.3) (end 139.73 122.3) (width 0.5) (layer F.Cu) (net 9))
 (segment (start 147.32 120.65) (end 153.67 120.65) (width 0.5) (layer F.Cu) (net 9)))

